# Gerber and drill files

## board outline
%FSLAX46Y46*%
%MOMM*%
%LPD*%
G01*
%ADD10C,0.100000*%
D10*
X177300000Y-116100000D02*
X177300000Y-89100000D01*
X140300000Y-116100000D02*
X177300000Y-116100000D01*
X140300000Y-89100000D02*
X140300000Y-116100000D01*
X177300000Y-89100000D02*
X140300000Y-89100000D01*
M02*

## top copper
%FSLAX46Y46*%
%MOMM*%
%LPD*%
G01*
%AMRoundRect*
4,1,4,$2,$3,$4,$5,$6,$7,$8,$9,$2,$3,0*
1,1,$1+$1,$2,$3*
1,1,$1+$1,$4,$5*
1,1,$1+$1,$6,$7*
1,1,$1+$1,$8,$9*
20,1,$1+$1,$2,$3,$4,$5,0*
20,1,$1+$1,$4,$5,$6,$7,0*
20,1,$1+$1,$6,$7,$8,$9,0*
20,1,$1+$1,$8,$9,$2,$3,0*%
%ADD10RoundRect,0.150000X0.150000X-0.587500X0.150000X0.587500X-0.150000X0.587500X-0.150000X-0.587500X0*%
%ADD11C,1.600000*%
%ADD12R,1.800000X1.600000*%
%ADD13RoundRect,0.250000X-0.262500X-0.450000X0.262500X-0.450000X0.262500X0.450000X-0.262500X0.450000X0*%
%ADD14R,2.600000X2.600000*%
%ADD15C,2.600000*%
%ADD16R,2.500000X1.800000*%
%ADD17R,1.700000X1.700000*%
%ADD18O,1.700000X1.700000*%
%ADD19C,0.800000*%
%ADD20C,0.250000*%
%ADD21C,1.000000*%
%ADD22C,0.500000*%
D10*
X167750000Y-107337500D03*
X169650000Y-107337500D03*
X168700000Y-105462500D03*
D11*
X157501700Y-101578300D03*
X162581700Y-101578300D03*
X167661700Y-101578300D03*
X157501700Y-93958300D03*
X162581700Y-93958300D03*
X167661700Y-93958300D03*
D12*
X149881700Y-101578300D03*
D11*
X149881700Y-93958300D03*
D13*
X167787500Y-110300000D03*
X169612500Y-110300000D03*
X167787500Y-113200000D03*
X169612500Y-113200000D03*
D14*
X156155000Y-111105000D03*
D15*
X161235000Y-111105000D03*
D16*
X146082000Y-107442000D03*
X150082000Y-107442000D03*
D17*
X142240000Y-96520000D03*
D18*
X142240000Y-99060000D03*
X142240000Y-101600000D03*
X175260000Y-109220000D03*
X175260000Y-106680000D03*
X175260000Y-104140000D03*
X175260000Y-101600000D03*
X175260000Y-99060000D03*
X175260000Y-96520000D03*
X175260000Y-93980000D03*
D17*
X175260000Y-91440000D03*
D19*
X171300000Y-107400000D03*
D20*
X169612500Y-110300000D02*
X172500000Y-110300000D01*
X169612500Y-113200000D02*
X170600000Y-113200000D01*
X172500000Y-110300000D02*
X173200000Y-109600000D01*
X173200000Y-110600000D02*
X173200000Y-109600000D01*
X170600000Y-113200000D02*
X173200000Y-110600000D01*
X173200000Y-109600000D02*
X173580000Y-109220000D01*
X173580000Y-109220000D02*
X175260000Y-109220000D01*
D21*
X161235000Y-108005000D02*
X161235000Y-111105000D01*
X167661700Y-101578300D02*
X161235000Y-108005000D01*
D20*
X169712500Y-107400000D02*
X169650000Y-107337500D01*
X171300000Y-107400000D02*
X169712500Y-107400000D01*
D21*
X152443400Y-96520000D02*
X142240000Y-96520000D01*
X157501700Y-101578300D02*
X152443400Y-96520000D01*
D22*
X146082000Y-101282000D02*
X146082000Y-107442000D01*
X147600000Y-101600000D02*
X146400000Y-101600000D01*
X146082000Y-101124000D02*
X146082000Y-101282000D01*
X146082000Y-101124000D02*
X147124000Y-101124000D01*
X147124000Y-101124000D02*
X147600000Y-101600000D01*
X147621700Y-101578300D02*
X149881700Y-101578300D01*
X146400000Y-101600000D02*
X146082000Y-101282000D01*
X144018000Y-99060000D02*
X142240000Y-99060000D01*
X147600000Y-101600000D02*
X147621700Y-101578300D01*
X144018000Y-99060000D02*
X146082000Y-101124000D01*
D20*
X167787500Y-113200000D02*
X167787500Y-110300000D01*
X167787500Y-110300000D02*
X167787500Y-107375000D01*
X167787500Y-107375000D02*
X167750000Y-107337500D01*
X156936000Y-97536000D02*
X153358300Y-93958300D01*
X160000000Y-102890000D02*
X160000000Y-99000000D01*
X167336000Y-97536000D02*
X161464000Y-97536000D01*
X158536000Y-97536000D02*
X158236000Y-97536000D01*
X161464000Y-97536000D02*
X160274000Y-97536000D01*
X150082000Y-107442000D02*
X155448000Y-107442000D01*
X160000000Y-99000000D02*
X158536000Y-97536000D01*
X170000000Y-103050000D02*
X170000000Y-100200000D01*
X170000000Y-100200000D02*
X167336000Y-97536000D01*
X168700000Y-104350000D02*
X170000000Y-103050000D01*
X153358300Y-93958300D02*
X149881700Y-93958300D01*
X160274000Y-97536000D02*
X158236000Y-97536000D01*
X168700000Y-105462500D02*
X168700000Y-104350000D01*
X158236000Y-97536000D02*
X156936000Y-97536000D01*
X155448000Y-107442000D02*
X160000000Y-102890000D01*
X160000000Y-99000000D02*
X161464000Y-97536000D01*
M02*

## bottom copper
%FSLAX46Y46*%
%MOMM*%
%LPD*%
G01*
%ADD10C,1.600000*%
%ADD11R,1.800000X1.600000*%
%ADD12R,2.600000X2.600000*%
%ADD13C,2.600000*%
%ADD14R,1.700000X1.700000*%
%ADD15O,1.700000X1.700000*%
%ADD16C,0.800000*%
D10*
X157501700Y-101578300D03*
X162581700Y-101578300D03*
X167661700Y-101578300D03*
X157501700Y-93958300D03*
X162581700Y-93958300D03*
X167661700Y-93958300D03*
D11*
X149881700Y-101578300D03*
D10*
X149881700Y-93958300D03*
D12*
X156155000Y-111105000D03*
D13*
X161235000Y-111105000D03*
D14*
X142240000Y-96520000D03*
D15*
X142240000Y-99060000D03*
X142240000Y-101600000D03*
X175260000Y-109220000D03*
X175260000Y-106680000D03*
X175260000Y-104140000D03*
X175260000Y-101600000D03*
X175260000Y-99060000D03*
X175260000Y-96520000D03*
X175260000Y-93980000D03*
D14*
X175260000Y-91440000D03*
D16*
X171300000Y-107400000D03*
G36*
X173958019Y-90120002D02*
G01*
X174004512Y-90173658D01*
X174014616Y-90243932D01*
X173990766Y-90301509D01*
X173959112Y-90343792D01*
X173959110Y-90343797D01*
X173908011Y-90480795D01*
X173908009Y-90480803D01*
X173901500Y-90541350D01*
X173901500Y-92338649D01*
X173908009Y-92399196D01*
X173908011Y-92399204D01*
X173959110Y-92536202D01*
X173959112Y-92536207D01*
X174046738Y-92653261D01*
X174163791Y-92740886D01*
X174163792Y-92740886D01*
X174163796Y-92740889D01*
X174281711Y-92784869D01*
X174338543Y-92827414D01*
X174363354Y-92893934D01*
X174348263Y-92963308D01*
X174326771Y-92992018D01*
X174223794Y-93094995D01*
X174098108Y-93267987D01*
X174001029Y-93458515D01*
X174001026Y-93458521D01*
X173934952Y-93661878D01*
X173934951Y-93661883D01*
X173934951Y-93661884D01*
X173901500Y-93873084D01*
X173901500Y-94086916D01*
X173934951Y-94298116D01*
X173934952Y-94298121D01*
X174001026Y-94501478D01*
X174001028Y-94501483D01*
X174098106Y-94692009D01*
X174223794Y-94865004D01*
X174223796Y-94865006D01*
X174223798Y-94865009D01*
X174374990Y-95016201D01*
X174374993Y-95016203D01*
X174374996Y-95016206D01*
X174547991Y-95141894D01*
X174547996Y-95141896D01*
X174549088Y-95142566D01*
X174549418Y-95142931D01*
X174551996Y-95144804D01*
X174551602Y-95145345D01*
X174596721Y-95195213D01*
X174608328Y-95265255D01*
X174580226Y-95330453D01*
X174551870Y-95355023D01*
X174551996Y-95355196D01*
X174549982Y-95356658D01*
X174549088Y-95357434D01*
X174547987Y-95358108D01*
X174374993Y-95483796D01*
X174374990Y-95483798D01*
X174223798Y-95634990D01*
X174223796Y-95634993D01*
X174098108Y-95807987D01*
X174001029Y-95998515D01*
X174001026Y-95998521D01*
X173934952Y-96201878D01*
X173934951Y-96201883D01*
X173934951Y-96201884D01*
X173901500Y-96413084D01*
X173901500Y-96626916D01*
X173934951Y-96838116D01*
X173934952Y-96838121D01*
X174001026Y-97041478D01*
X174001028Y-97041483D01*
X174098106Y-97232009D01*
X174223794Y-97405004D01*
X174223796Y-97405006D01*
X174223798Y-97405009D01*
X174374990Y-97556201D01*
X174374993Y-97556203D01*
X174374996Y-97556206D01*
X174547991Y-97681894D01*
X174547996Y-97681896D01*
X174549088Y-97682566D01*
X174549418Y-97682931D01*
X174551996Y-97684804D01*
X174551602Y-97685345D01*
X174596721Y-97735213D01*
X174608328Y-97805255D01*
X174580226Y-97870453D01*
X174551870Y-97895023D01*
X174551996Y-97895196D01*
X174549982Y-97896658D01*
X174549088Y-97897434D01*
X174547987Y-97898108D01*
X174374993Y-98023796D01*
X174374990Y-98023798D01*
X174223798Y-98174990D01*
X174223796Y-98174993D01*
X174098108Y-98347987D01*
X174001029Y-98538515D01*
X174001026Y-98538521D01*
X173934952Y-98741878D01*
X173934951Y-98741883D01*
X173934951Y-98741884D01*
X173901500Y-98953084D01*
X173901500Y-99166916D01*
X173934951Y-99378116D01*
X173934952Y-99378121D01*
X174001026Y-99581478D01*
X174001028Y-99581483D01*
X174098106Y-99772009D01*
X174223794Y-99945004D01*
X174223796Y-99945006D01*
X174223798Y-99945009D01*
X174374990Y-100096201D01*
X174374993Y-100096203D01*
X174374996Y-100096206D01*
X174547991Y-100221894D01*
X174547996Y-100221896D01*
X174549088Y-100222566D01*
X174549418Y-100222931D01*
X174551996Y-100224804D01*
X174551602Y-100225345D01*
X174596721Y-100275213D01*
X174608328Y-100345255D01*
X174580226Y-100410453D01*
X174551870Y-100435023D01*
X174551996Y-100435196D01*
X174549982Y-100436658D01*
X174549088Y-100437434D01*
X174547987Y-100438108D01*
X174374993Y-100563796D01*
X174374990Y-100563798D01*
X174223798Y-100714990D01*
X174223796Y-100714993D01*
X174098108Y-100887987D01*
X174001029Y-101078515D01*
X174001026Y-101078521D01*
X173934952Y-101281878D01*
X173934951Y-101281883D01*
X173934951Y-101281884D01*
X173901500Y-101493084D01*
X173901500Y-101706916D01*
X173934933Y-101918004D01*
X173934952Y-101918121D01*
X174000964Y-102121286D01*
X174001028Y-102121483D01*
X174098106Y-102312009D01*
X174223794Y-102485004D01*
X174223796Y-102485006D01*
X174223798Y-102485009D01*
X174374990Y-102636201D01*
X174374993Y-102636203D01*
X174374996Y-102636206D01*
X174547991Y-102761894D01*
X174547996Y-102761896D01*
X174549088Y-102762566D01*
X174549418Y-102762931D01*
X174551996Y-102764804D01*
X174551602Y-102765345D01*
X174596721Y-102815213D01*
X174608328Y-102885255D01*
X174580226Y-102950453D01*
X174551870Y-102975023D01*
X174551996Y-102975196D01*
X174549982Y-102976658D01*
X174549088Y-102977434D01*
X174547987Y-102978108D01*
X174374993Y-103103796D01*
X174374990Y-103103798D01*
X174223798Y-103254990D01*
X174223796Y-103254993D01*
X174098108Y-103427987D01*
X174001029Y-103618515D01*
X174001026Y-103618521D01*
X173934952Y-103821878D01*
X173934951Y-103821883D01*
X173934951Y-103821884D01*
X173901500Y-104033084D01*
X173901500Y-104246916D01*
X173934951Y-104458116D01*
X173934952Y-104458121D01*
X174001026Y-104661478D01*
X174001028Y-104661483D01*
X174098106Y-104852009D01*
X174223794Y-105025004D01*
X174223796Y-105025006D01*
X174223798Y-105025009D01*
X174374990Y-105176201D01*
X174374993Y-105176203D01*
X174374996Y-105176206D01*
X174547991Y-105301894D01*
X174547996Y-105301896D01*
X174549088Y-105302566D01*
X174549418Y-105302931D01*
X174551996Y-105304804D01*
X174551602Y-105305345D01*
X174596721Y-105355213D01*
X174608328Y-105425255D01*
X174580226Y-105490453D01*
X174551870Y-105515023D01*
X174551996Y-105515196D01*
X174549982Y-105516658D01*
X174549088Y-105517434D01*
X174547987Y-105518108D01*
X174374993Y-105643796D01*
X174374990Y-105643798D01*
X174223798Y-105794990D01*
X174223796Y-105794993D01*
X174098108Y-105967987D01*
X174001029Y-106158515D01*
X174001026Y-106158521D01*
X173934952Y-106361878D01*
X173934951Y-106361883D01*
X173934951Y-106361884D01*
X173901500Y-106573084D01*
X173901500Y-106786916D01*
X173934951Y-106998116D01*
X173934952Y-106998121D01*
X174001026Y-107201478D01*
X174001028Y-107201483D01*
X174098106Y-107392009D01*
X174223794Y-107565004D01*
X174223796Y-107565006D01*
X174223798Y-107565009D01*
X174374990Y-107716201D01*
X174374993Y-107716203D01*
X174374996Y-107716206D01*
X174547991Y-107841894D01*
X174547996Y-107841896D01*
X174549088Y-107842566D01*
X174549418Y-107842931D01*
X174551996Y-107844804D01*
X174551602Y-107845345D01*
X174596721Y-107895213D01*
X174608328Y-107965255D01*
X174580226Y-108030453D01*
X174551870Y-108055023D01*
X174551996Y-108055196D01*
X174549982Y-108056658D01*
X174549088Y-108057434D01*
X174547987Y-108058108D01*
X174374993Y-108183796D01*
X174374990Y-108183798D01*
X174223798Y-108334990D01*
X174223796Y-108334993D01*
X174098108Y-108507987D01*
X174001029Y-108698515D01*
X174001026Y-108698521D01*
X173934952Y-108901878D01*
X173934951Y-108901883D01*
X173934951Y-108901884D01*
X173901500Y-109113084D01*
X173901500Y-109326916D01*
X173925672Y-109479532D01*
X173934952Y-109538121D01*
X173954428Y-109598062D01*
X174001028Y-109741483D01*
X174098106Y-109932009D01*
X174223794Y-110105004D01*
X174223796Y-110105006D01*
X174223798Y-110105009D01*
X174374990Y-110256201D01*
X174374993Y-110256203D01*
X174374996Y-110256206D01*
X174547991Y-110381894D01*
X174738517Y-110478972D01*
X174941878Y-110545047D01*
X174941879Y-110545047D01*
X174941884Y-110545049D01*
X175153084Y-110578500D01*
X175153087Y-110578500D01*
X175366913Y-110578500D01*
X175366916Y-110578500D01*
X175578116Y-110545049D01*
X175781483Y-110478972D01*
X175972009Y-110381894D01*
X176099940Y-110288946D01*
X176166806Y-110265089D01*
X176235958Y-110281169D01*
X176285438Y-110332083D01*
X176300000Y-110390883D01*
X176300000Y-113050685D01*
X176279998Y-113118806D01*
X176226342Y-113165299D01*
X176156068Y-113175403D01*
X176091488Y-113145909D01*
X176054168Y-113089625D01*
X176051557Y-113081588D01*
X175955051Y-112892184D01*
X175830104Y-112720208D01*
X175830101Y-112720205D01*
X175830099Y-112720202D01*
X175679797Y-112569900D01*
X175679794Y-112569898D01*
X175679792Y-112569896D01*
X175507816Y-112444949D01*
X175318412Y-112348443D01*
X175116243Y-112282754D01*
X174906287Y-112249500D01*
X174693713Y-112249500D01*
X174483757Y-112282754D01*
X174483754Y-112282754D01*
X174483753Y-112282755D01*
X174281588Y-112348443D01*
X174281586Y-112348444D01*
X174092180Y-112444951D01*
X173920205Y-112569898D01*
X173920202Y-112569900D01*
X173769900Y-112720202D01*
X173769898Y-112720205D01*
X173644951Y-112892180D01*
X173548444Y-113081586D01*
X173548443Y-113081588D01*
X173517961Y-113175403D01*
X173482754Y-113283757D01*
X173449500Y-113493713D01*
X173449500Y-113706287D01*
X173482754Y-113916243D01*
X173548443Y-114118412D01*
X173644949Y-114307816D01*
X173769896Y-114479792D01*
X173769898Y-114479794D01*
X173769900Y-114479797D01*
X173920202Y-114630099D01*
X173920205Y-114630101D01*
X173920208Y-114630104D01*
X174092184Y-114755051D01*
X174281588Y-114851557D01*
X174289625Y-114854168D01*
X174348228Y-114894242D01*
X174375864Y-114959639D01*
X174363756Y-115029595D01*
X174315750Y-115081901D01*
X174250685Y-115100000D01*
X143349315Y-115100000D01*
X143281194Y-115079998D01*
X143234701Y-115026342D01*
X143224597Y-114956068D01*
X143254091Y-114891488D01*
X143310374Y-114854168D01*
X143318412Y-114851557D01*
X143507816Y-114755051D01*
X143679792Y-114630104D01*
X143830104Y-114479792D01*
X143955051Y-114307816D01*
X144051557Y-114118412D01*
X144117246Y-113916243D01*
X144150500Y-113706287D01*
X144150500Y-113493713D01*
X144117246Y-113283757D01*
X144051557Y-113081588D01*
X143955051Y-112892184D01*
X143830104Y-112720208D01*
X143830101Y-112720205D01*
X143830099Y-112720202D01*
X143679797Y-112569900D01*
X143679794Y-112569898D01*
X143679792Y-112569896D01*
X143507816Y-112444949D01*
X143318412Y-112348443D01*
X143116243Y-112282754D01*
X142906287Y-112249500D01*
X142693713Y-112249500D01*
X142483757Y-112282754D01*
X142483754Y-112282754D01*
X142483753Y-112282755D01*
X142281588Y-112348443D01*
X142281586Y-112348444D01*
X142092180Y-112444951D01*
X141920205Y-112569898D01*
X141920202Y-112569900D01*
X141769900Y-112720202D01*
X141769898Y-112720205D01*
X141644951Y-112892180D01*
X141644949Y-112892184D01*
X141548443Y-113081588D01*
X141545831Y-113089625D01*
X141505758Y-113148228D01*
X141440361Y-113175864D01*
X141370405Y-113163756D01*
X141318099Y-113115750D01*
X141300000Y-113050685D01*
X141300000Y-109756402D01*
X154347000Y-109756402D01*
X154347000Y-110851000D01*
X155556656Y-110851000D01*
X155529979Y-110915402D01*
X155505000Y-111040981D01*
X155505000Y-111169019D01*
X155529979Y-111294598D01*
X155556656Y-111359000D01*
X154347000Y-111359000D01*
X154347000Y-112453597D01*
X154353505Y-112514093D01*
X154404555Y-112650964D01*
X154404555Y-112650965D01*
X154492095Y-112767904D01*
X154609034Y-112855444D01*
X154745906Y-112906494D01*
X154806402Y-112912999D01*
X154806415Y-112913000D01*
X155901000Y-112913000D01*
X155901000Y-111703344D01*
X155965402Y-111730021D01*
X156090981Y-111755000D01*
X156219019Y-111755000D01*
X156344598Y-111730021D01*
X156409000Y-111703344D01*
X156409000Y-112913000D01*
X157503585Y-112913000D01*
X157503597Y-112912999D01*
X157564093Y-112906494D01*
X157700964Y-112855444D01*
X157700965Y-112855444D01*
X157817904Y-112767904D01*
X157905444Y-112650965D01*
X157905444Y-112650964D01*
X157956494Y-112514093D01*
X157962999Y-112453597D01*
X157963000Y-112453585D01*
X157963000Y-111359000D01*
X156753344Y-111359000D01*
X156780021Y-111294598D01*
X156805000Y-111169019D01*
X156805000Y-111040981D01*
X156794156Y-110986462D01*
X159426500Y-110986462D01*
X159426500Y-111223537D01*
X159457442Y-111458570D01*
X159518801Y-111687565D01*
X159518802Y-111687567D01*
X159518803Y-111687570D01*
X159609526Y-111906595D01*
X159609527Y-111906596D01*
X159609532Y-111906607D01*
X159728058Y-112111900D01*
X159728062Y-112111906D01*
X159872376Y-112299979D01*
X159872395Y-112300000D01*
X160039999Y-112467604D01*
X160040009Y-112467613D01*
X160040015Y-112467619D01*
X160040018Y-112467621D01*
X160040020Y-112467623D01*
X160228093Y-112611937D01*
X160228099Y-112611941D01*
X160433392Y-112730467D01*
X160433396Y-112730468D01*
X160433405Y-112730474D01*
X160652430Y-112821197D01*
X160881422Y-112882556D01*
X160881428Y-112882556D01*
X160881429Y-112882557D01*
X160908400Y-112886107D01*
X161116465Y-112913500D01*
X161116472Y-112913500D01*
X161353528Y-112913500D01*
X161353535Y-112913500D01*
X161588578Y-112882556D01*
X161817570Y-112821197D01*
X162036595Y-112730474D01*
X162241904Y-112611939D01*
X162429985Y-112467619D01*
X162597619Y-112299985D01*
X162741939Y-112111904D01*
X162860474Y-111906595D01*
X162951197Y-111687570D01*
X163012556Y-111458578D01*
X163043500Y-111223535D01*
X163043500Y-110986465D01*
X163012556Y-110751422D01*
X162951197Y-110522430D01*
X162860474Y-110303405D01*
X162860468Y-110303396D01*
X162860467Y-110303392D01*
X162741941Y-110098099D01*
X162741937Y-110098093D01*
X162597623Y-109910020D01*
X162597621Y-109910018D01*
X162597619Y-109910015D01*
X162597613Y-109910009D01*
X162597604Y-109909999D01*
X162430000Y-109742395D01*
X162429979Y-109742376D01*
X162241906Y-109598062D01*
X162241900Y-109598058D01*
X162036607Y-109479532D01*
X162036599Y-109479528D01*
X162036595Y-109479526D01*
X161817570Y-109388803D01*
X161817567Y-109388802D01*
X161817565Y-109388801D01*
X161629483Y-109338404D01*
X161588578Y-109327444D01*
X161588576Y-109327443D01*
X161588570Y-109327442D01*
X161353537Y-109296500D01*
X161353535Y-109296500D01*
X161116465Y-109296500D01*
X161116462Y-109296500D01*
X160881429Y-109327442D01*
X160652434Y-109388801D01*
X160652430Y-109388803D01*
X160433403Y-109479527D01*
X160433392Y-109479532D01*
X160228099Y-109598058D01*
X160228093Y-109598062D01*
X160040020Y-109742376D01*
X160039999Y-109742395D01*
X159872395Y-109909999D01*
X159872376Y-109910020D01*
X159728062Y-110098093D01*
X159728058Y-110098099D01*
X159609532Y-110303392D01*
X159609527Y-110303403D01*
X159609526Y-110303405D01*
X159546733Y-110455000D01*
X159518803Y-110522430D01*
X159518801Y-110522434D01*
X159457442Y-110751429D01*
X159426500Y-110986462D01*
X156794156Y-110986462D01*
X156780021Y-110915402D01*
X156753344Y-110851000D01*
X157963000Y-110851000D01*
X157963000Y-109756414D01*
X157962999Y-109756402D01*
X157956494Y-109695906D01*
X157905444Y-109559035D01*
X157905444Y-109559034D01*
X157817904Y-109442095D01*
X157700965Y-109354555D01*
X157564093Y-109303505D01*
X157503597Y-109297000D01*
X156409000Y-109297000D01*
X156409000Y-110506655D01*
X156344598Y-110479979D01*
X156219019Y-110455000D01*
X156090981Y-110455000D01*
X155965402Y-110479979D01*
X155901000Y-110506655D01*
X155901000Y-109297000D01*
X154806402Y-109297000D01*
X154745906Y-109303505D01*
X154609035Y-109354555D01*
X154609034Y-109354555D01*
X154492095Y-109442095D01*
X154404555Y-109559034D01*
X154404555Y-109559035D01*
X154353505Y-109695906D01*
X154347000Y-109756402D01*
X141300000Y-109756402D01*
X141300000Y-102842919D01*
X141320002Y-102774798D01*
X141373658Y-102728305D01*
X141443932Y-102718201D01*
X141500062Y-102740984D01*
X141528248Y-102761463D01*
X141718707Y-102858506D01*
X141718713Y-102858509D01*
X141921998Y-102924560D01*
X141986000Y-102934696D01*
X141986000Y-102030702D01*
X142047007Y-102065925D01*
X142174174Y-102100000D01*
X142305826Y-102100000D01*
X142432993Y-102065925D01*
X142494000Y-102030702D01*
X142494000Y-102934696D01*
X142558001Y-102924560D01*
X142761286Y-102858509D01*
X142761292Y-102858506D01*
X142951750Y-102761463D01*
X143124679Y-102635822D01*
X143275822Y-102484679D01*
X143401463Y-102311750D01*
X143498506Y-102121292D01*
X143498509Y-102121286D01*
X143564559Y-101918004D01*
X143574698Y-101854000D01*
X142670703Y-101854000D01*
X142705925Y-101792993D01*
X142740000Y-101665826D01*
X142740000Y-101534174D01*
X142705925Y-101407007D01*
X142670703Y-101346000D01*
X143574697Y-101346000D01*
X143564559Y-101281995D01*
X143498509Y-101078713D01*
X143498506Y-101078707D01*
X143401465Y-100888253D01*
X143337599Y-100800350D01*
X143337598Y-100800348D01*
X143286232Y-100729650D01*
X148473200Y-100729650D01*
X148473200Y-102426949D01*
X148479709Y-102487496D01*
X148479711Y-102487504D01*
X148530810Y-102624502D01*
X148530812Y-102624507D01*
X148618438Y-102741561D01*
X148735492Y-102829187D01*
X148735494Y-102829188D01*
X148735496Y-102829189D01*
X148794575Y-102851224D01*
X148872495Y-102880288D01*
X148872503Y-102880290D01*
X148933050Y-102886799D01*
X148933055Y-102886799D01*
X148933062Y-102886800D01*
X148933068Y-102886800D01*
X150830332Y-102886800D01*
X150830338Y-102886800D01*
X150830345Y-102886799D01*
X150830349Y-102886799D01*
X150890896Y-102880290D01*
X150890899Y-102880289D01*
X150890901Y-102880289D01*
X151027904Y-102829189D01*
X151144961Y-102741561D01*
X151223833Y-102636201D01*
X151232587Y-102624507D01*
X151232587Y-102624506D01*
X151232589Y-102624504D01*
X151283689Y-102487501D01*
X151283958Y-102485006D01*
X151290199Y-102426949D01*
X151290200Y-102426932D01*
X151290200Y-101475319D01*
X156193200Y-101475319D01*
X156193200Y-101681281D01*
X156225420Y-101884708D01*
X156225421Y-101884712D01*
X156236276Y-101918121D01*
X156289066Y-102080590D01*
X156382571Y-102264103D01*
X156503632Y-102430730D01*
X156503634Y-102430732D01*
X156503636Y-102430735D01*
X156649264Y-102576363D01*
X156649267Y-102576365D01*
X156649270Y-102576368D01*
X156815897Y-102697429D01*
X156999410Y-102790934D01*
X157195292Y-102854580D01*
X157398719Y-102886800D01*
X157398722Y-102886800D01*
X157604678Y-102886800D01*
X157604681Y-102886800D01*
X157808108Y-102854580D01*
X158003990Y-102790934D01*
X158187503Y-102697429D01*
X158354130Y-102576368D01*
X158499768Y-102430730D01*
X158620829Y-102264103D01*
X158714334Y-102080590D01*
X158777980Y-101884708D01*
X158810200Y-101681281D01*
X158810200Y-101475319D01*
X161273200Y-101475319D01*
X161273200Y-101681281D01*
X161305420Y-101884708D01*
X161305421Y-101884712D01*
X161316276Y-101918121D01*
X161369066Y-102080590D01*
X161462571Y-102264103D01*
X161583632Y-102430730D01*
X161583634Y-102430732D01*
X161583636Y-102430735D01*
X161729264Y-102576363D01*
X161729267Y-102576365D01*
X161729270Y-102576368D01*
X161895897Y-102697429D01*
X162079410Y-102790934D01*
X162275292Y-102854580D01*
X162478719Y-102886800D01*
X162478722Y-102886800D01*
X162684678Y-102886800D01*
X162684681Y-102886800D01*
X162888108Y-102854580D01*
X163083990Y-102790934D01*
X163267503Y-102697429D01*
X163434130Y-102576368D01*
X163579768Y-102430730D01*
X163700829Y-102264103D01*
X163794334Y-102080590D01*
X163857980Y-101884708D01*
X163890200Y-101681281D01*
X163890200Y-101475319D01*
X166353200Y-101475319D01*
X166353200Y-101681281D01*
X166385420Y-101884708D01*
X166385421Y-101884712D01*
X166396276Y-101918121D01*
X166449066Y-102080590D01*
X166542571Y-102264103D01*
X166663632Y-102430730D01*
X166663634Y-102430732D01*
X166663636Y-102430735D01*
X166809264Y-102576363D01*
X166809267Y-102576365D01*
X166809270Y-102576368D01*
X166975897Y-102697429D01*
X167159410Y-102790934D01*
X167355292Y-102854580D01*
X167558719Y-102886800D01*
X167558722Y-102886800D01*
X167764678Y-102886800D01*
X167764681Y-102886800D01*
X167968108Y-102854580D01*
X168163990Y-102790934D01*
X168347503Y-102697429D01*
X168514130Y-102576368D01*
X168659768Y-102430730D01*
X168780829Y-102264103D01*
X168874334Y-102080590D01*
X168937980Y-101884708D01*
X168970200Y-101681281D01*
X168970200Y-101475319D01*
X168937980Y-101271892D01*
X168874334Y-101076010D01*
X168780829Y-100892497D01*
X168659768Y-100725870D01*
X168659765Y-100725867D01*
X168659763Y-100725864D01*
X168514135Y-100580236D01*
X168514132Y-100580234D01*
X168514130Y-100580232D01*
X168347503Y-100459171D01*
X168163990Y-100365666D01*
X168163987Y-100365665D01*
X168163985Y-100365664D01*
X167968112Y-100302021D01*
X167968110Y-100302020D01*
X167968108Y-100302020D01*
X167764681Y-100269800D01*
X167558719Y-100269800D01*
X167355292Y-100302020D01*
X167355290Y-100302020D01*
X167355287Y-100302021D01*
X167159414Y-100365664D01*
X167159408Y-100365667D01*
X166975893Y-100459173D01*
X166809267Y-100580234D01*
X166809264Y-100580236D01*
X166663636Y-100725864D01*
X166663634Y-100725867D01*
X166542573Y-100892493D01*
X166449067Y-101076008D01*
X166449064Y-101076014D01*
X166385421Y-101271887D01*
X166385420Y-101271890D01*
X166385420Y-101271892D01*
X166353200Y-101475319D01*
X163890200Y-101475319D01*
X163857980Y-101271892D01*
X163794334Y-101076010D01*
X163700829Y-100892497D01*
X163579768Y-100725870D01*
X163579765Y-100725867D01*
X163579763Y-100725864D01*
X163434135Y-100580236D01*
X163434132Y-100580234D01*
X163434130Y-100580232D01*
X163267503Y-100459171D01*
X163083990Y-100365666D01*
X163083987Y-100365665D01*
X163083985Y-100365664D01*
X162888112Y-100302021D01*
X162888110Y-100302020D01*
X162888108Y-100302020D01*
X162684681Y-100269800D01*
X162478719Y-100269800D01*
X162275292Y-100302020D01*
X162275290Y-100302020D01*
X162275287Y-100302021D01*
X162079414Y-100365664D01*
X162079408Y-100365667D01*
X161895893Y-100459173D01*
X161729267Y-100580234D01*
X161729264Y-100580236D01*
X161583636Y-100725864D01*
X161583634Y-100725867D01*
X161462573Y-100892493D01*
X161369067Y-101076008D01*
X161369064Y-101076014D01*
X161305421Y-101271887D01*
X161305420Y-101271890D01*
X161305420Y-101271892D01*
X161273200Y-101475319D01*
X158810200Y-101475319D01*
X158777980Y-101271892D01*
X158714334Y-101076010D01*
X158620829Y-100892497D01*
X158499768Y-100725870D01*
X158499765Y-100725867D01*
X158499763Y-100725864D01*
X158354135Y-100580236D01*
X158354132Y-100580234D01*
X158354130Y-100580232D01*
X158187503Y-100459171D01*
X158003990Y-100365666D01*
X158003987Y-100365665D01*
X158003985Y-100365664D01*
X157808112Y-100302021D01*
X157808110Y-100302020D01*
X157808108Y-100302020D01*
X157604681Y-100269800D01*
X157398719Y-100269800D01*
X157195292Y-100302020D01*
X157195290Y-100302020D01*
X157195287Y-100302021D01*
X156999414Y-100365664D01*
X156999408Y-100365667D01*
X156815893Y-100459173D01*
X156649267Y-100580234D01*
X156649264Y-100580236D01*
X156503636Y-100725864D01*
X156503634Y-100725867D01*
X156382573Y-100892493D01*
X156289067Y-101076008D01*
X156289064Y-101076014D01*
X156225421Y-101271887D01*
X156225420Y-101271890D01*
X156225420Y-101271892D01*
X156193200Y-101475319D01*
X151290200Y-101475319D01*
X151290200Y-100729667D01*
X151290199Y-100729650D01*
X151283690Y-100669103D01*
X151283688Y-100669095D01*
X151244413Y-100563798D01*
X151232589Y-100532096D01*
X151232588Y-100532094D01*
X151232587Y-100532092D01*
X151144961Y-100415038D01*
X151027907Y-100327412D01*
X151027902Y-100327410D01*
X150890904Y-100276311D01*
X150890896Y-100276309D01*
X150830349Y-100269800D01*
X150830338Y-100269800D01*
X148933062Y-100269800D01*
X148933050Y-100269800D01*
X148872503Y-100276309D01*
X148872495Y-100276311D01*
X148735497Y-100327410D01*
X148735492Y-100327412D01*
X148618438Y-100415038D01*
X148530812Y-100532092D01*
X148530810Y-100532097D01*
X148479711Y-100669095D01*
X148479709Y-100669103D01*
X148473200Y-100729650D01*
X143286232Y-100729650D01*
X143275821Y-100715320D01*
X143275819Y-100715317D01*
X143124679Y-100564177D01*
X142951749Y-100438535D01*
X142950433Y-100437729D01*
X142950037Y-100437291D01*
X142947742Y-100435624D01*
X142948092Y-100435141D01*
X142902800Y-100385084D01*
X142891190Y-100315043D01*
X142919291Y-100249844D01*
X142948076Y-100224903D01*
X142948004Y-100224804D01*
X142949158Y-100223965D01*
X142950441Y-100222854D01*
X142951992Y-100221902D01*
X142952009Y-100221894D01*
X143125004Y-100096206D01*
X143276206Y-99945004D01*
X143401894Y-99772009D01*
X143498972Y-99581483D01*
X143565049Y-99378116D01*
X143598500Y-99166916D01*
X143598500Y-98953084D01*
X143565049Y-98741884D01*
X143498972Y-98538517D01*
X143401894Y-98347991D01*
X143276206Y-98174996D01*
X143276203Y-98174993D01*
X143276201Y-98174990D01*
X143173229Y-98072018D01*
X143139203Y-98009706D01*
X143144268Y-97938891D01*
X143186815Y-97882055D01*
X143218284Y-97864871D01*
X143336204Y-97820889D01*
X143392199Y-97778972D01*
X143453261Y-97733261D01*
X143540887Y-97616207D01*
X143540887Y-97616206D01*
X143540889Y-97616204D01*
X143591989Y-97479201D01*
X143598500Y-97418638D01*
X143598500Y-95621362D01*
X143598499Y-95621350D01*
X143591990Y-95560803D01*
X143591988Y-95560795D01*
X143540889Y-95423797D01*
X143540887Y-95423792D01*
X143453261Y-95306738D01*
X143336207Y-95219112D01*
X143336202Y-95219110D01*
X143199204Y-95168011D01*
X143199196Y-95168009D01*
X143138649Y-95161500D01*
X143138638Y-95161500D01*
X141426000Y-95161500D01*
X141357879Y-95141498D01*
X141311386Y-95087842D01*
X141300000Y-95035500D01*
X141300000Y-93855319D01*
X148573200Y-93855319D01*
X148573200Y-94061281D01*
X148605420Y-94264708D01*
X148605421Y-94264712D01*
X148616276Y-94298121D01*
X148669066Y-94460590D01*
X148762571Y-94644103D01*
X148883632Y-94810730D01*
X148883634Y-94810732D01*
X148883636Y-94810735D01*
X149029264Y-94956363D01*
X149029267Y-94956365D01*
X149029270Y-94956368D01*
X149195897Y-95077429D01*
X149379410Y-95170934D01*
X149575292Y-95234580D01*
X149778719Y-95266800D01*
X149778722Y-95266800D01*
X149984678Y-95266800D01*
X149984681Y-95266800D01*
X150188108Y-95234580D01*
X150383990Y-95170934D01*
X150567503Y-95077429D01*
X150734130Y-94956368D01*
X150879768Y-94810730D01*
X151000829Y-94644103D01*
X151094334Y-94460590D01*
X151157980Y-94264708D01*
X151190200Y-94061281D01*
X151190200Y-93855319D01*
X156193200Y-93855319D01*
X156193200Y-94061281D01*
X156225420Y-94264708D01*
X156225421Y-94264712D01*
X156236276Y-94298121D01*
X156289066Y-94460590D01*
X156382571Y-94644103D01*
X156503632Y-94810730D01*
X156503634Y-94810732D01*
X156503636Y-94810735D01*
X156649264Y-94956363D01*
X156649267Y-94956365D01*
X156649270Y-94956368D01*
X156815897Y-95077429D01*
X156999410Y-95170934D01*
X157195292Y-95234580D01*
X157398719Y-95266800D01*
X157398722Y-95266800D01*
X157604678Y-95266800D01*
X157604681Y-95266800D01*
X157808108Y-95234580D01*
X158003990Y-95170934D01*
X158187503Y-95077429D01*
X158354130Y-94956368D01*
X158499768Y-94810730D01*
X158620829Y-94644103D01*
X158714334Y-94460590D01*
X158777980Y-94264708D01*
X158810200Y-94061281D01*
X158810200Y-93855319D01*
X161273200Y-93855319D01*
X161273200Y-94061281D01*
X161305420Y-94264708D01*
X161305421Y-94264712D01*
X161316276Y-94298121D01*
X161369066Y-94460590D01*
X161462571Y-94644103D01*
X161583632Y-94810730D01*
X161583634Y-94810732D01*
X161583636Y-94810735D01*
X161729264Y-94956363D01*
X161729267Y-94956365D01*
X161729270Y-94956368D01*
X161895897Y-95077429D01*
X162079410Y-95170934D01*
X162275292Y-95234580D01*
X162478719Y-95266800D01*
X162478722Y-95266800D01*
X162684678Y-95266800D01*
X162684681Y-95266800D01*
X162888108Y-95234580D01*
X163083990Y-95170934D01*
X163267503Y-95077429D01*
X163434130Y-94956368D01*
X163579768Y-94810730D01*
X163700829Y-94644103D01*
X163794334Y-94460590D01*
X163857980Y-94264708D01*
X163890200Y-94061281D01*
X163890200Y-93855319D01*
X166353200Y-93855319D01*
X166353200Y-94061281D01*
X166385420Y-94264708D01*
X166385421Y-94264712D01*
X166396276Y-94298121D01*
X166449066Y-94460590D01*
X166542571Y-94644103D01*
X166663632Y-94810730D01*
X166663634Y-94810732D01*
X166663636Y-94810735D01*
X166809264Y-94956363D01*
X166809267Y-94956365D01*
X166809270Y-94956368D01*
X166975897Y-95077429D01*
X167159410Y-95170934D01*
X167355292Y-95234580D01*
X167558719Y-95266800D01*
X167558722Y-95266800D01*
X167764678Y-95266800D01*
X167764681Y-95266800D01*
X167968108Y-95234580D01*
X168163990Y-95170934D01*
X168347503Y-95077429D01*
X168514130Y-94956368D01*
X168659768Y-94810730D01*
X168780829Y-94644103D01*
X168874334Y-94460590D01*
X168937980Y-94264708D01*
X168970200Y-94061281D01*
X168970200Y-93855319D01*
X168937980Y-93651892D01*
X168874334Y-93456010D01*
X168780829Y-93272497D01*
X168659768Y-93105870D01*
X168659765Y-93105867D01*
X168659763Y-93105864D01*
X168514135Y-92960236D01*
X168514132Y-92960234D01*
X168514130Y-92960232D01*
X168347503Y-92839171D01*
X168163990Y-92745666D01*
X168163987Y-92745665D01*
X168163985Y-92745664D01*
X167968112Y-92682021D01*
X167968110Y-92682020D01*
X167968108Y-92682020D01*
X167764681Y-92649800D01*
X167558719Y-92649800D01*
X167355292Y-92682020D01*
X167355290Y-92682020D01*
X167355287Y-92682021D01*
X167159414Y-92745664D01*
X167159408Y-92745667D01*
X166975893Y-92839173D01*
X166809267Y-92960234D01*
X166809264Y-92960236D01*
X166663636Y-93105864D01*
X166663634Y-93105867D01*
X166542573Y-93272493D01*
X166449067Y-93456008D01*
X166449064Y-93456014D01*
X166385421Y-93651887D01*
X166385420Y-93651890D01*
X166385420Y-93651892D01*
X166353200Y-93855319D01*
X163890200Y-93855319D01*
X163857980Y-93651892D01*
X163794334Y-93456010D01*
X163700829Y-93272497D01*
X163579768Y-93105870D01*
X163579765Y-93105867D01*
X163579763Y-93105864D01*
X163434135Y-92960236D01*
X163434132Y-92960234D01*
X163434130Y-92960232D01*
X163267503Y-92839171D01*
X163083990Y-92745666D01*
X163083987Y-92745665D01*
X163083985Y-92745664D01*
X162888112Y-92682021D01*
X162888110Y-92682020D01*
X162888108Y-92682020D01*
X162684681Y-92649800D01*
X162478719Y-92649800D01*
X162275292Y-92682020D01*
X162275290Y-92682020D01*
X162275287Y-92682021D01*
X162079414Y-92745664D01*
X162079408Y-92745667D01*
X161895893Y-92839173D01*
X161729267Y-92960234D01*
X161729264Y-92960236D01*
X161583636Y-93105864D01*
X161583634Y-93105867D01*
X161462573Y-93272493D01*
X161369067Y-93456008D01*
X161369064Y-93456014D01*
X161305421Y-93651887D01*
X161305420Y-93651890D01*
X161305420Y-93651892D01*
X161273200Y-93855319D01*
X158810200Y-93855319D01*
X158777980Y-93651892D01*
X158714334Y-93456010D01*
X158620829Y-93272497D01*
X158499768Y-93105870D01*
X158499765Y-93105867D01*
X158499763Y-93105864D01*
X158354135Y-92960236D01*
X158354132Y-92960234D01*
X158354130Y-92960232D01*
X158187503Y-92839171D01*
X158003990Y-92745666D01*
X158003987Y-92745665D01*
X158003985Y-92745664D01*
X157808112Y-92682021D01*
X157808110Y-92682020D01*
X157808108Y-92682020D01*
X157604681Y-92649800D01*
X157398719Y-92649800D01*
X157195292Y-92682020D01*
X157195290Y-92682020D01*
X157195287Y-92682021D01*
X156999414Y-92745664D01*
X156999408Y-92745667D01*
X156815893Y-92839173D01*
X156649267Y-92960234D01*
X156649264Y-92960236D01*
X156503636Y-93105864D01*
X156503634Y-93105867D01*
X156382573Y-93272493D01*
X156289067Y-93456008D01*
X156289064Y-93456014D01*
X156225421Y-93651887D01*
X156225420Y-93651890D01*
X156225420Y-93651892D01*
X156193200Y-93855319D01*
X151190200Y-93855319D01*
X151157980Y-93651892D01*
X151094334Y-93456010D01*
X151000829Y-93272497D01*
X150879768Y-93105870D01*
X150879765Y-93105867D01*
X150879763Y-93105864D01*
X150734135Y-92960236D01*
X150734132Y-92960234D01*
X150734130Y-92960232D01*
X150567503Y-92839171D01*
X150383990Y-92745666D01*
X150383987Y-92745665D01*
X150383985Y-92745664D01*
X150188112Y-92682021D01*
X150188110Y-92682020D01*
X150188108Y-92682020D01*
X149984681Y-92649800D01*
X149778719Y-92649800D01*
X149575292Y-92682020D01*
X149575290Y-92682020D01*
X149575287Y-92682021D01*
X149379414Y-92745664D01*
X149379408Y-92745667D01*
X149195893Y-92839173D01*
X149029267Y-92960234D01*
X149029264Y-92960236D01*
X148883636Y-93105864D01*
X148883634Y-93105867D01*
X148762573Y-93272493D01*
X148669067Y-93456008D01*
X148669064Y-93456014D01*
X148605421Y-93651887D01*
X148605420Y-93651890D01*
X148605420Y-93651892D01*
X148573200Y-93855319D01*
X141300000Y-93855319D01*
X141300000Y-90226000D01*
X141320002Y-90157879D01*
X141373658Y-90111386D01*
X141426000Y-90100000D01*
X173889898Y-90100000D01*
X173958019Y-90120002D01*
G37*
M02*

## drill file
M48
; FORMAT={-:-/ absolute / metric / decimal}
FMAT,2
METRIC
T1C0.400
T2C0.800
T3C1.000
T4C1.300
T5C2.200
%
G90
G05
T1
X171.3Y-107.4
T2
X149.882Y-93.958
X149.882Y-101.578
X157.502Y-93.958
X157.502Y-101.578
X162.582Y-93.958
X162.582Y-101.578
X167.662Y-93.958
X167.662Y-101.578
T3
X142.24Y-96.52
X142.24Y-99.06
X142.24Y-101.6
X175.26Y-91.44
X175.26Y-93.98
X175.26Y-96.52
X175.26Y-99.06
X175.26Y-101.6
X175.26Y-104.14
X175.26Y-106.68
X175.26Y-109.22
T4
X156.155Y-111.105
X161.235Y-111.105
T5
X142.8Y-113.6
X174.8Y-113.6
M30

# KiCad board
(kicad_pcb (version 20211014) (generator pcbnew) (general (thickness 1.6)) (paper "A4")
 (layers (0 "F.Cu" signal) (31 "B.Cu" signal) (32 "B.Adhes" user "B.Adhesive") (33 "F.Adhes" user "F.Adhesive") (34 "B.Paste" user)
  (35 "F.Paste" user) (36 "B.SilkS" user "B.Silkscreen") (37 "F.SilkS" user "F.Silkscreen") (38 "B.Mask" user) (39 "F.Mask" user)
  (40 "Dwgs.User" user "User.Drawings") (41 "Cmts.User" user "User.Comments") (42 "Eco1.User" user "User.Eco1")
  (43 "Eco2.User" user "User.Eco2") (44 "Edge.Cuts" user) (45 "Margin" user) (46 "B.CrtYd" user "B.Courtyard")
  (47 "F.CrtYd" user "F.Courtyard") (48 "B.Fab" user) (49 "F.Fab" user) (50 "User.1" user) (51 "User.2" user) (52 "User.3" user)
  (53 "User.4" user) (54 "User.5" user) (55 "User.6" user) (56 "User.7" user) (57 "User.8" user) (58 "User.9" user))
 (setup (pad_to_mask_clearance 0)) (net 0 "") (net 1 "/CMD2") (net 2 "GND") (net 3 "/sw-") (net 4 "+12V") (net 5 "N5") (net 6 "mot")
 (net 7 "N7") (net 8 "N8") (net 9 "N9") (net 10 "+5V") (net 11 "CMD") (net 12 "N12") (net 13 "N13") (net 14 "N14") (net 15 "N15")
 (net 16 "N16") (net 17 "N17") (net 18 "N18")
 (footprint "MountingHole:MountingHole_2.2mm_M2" (layer "F.Cu") (at 174.8 113.6)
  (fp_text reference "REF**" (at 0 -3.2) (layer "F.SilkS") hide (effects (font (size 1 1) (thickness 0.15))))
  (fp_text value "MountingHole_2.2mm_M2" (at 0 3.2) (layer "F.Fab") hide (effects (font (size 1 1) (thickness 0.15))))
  (pad "" np_thru_hole circle (at 0 0) (size 2.2 2.2) (drill 2.2) (layers F&B.Cu *.Mask)))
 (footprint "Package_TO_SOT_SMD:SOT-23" (layer "F.Cu") (at 168.7 106.4 90)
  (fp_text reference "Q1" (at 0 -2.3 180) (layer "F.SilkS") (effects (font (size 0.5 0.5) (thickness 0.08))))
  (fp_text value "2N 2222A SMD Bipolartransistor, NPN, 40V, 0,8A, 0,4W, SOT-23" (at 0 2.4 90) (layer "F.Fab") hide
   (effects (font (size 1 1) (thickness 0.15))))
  (pad "1" smd roundrect (at -0.9375 -0.95 90) (size 1.475 0.6) (layers "F.Cu" "F.Paste" "F.Mask") (roundrect_rratio 0.25) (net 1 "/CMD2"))
  (pad "2" smd roundrect (at -0.9375 0.95 90) (size 1.475 0.6) (layers "F.Cu" "F.Paste" "F.Mask") (roundrect_rratio 0.25) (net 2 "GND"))
  (pad "3" smd roundrect (at 0.9375 0 90) (size 1.475 0.6) (layers "F.Cu" "F.Paste" "F.Mask") (roundrect_rratio 0.25) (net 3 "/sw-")))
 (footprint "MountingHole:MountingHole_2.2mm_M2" (layer "F.Cu") (at 142.8 113.6)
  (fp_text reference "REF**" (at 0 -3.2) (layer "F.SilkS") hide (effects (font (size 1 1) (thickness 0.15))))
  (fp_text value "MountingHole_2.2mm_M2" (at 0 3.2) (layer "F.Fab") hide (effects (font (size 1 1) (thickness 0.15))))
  (pad "" np_thru_hole circle (at 0 0) (size 2.2 2.2) (drill 2.2) (layers F&B.Cu *.Mask)))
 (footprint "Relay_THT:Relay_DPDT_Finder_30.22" (layer "F.Cu") (at 149.8817 101.5783)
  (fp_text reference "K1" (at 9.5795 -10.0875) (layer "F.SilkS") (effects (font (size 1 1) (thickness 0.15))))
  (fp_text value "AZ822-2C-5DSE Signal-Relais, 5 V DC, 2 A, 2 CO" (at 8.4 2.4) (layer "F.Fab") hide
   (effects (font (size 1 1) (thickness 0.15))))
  (pad "11" thru_hole circle (at 7.62 0 90) (size 1.6 1.6) (drill 0.8) (layers *.Cu *.Mask) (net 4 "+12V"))
  (pad "12" thru_hole circle (at 12.7 0 90) (size 1.6 1.6) (drill 0.8) (layers *.Cu *.Mask) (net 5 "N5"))
  (pad "14" thru_hole circle (at 17.78 0 90) (size 1.6 1.6) (drill 0.8) (layers *.Cu *.Mask) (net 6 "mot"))
  (pad "21" thru_hole circle (at 7.62 -7.62 90) (size 1.6 1.6) (drill 0.8) (layers *.Cu *.Mask) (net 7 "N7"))
  (pad "22" thru_hole circle (at 12.7 -7.62 90) (size 1.6 1.6) (drill 0.8) (layers *.Cu *.Mask) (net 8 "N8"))
  (pad "24" thru_hole circle (at 17.78 -7.62 180) (size 1.6 1.6) (drill 0.8) (layers *.Cu *.Mask) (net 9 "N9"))
  (pad "A1" thru_hole rect (at 0 0 90) (size 1.6 1.8) (drill 0.8) (layers *.Cu *.Mask) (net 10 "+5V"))
  (pad "A2" thru_hole circle (at 0 -7.62 90) (size 1.6 1.6) (drill 0.8) (layers *.Cu *.Mask) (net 3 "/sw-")))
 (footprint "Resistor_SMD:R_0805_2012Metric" (layer "F.Cu") (at 168.7 110.3)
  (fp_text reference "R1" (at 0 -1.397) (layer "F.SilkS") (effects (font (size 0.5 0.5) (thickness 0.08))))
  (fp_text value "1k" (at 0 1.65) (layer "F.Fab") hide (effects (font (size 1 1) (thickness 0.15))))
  (pad "1" smd roundrect (at -0.9125 0) (size 1.025 1.4) (layers "F.Cu" "F.Paste" "F.Mask") (roundrect_rratio 0.243902) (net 1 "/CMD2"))
  (pad "2" smd roundrect (at 0.9125 0) (size 1.025 1.4) (layers "F.Cu" "F.Paste" "F.Mask") (roundrect_rratio 0.243902) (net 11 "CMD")))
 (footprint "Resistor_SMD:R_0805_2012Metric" (layer "F.Cu") (at 168.7 113.2)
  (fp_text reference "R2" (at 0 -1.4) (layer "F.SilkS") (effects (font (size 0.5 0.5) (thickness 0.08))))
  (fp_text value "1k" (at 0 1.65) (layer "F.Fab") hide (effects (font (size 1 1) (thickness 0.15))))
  (pad "1" smd roundrect (at -0.9125 0) (size 1.025 1.4) (layers "F.Cu" "F.Paste" "F.Mask") (roundrect_rratio 0.243902) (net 1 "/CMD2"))
  (pad "2" smd roundrect (at 0.9125 0) (size 1.025 1.4) (layers "F.Cu" "F.Paste" "F.Mask") (roundrect_rratio 0.243902) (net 11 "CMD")))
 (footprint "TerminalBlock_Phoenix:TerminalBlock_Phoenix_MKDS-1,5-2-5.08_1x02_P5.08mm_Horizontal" (layer "F.Cu") (at 156.155 111.105)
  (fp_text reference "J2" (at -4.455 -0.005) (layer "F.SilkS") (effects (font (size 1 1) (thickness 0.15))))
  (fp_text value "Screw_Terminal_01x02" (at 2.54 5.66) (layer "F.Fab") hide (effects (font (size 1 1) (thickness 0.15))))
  (pad "1" thru_hole rect (at 0 0) (size 2.6 2.6) (drill 1.3) (layers *.Cu *.Mask) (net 2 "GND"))
  (pad "2" thru_hole circle (at 5.08 0) (size 2.6 2.6) (drill 1.3) (layers *.Cu *.Mask) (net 6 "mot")))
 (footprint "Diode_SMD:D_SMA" (layer "F.Cu") (at 148.082 107.442)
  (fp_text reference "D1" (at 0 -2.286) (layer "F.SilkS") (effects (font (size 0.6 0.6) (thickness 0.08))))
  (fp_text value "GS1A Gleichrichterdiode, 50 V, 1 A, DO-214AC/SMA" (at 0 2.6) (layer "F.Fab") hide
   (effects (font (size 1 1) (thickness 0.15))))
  (pad "1" smd rect (at -2 0) (size 2.5 1.8) (layers "F.Cu" "F.Paste" "F.Mask") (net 10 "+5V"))
  (pad "2" smd rect (at 2 0) (size 2.5 1.8) (layers "F.Cu" "F.Paste" "F.Mask") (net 3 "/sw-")))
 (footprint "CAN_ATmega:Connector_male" (layer "F.Cu") (at 157.48 99.06)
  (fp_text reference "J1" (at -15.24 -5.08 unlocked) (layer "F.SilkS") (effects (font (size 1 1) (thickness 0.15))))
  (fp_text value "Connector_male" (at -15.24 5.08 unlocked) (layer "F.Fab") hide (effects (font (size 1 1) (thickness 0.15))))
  (pad "1" thru_hole rect (at -15.24 -2.54) (size 1.7 1.7) (drill 1) (layers *.Cu *.Mask) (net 4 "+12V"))
  (pad "2" thru_hole oval (at -15.24 0) (size 1.7 1.7) (drill 1) (layers *.Cu *.Mask) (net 10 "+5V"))
  (pad "3" thru_hole oval (at -15.24 2.54) (size 1.7 1.7) (drill 1) (layers *.Cu *.Mask) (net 2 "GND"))
  (pad "4" thru_hole oval (at 17.78 10.16) (size 1.7 1.7) (drill 1) (layers *.Cu *.Mask) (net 11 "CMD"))
  (pad "5" thru_hole oval (at 17.78 7.62) (size 1.7 1.7) (drill 1) (layers *.Cu *.Mask) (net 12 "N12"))
  (pad "6" thru_hole oval (at 17.78 5.08) (size 1.7 1.7) (drill 1) (layers *.Cu *.Mask) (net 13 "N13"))
  (pad "7" thru_hole oval (at 17.78 2.54) (size 1.7 1.7) (drill 1) (layers *.Cu *.Mask) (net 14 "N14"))
  (pad "8" thru_hole oval (at 17.78 0) (size 1.7 1.7) (drill 1) (layers *.Cu *.Mask) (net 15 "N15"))
  (pad "9" thru_hole oval (at 17.78 -2.54) (size 1.7 1.7) (drill 1) (layers *.Cu *.Mask) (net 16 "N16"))
  (pad "10" thru_hole oval (at 17.78 -5.08) (size 1.7 1.7) (drill 1) (layers *.Cu *.Mask) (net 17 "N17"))
  (pad "11" thru_hole rect (at 17.78 -7.62) (size 1.7 1.7) (drill 1) (layers *.Cu *.Mask) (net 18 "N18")))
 (gr_line (start 177.3 116.1) (end 177.3 89.1) (layer "Edge.Cuts") (width 0.1))
 (gr_line (start 140.3 116.1) (end 177.3 116.1) (layer "Edge.Cuts") (width 0.1))
 (gr_line (start 140.3 89.1) (end 140.3 116.1) (layer "Edge.Cuts") (width 0.1))
 (gr_line (start 177.3 89.1) (end 140.3 89.1) (layer "Edge.Cuts") (width 0.1))
 (segment (start 169.6125 110.3) (end 172.5 110.3) (width 0.25) (layer "F.Cu") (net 11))
 (segment (start 169.6125 113.2) (end 170.6 113.2) (width 0.25) (layer "F.Cu") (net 11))
 (segment (start 172.5 110.3) (end 173.2 109.6) (width 0.25) (layer "F.Cu") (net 11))
 (segment (start 173.2 110.6) (end 173.2 109.6) (width 0.25) (layer "F.Cu") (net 11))
 (segment (start 170.6 113.2) (end 173.2 110.6) (width 0.25) (layer "F.Cu") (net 11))
 (segment (start 173.2 109.6) (end 173.58 109.22) (width 0.25) (layer "F.Cu") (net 11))
 (segment (start 173.58 109.22) (end 175.26 109.22) (width 0.25) (layer "F.Cu") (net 11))
 (segment (start 161.235 108.005) (end 161.235 111.105) (width 1) (layer "F.Cu") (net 6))
 (segment (start 167.6617 101.5783) (end 161.235 108.005) (width 1) (layer "F.Cu") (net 6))
 (segment (start 169.7125 107.4) (end 169.65 107.3375) (width 0.25) (layer "F.Cu") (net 2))
 (segment (start 171.3 107.4) (end 169.7125 107.4) (width 0.25) (layer "F.Cu") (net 2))
 (via (at 171.3 107.4) (size 0.8) (drill 0.4) (layers "F.Cu" "B.Cu") (free) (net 2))
 (segment (start 152.4434 96.52) (end 142.24 96.52) (width 1) (layer "F.Cu") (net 4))
 (segment (start 157.5017 101.5783) (end 152.4434 96.52) (width 1) (layer "F.Cu") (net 4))
 (segment (start 146.082 101.282) (end 146.082 107.442) (width 0.5) (layer "F.Cu") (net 10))
 (segment (start 147.6 101.6) (end 146.4 101.6) (width 0.5) (layer "F.Cu") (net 10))
 (segment (start 146.082 101.124) (end 146.082 101.282) (width 0.5) (layer "F.Cu") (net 10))
 (segment (start 146.082 101.124) (end 147.124 101.124) (width 0.5) (layer "F.Cu") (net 10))
 (segment (start 147.124 101.124) (end 147.6 101.6) (width 0.5) (layer "F.Cu") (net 10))
 (segment (start 147.6217 101.5783) (end 149.8817 101.5783) (width 0.5) (layer "F.Cu") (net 10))
 (segment (start 146.4 101.6) (end 146.082 101.282) (width 0.5) (layer "F.Cu") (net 10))
 (segment (start 144.018 99.06) (end 142.24 99.06) (width 0.5) (layer "F.Cu") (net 10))
 (segment (start 147.6 101.6) (end 147.6217 101.5783) (width 0.5) (layer "F.Cu") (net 10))
 (segment (start 144.018 99.06) (end 146.082 101.124) (width 0.5) (layer "F.Cu") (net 10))
 (segment (start 167.7875 113.2) (end 167.7875 110.3) (width 0.25) (layer "F.Cu") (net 1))
 (segment (start 167.7875 110.3) (end 167.7875 107.375) (width 0.25) (layer "F.Cu") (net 1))
 (segment (start 167.7875 107.375) (end 167.75 107.3375) (width 0.25) (layer "F.Cu") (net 1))
 (segment (start 156.936 97.536) (end 153.3583 93.9583) (width 0.25) (layer "F.Cu") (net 3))
 (segment (start 160 102.89) (end 160 99) (width 0.25) (layer "F.Cu") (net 3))
 (segment (start 167.336 97.536) (end 161.464 97.536) (width 0.25) (layer "F.Cu") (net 3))
 (segment (start 158.536 97.536) (end 158.236 97.536) (width 0.25) (layer "F.Cu") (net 3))
 (segment (start 161.464 97.536) (end 160.274 97.536) (width 0.25) (layer "F.Cu") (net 3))
 (segment (start 150.082 107.442) (end 155.448 107.442) (width 0.25) (layer "F.Cu") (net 3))
 (segment (start 160 99) (end 158.536 97.536) (width 0.25) (layer "F.Cu") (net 3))
 (segment (start 170 103.05) (end 170 100.2) (width 0.25) (layer "F.Cu") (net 3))
 (segment (start 170 100.2) (end 167.336 97.536) (width 0.25) (layer "F.Cu") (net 3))
 (segment (start 168.7 104.35) (end 170 103.05) (width 0.25) (layer "F.Cu") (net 3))
 (segment (start 153.3583 93.9583) (end 149.8817 93.9583) (width 0.25) (layer "F.Cu") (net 3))
 (segment (start 160.274 97.536) (end 158.236 97.536) (width 0.25) (layer "F.Cu") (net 3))
 (segment (start 168.7 105.4625) (end 168.7 104.35) (width 0.25) (layer "F.Cu") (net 3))
 (segment (start 158.236 97.536) (end 156.936 97.536) (width 0.25) (layer "F.Cu") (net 3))
 (segment (start 155.448 107.442) (end 160 102.89) (width 0.25) (layer "F.Cu") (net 3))
 (segment (start 160 99) (end 161.464 97.536) (width 0.25) (layer "F.Cu") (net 3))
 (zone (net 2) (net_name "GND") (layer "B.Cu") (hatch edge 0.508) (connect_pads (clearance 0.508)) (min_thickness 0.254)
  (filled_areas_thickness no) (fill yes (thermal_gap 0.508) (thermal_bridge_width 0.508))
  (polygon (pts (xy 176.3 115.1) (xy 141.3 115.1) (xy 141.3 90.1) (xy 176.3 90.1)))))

